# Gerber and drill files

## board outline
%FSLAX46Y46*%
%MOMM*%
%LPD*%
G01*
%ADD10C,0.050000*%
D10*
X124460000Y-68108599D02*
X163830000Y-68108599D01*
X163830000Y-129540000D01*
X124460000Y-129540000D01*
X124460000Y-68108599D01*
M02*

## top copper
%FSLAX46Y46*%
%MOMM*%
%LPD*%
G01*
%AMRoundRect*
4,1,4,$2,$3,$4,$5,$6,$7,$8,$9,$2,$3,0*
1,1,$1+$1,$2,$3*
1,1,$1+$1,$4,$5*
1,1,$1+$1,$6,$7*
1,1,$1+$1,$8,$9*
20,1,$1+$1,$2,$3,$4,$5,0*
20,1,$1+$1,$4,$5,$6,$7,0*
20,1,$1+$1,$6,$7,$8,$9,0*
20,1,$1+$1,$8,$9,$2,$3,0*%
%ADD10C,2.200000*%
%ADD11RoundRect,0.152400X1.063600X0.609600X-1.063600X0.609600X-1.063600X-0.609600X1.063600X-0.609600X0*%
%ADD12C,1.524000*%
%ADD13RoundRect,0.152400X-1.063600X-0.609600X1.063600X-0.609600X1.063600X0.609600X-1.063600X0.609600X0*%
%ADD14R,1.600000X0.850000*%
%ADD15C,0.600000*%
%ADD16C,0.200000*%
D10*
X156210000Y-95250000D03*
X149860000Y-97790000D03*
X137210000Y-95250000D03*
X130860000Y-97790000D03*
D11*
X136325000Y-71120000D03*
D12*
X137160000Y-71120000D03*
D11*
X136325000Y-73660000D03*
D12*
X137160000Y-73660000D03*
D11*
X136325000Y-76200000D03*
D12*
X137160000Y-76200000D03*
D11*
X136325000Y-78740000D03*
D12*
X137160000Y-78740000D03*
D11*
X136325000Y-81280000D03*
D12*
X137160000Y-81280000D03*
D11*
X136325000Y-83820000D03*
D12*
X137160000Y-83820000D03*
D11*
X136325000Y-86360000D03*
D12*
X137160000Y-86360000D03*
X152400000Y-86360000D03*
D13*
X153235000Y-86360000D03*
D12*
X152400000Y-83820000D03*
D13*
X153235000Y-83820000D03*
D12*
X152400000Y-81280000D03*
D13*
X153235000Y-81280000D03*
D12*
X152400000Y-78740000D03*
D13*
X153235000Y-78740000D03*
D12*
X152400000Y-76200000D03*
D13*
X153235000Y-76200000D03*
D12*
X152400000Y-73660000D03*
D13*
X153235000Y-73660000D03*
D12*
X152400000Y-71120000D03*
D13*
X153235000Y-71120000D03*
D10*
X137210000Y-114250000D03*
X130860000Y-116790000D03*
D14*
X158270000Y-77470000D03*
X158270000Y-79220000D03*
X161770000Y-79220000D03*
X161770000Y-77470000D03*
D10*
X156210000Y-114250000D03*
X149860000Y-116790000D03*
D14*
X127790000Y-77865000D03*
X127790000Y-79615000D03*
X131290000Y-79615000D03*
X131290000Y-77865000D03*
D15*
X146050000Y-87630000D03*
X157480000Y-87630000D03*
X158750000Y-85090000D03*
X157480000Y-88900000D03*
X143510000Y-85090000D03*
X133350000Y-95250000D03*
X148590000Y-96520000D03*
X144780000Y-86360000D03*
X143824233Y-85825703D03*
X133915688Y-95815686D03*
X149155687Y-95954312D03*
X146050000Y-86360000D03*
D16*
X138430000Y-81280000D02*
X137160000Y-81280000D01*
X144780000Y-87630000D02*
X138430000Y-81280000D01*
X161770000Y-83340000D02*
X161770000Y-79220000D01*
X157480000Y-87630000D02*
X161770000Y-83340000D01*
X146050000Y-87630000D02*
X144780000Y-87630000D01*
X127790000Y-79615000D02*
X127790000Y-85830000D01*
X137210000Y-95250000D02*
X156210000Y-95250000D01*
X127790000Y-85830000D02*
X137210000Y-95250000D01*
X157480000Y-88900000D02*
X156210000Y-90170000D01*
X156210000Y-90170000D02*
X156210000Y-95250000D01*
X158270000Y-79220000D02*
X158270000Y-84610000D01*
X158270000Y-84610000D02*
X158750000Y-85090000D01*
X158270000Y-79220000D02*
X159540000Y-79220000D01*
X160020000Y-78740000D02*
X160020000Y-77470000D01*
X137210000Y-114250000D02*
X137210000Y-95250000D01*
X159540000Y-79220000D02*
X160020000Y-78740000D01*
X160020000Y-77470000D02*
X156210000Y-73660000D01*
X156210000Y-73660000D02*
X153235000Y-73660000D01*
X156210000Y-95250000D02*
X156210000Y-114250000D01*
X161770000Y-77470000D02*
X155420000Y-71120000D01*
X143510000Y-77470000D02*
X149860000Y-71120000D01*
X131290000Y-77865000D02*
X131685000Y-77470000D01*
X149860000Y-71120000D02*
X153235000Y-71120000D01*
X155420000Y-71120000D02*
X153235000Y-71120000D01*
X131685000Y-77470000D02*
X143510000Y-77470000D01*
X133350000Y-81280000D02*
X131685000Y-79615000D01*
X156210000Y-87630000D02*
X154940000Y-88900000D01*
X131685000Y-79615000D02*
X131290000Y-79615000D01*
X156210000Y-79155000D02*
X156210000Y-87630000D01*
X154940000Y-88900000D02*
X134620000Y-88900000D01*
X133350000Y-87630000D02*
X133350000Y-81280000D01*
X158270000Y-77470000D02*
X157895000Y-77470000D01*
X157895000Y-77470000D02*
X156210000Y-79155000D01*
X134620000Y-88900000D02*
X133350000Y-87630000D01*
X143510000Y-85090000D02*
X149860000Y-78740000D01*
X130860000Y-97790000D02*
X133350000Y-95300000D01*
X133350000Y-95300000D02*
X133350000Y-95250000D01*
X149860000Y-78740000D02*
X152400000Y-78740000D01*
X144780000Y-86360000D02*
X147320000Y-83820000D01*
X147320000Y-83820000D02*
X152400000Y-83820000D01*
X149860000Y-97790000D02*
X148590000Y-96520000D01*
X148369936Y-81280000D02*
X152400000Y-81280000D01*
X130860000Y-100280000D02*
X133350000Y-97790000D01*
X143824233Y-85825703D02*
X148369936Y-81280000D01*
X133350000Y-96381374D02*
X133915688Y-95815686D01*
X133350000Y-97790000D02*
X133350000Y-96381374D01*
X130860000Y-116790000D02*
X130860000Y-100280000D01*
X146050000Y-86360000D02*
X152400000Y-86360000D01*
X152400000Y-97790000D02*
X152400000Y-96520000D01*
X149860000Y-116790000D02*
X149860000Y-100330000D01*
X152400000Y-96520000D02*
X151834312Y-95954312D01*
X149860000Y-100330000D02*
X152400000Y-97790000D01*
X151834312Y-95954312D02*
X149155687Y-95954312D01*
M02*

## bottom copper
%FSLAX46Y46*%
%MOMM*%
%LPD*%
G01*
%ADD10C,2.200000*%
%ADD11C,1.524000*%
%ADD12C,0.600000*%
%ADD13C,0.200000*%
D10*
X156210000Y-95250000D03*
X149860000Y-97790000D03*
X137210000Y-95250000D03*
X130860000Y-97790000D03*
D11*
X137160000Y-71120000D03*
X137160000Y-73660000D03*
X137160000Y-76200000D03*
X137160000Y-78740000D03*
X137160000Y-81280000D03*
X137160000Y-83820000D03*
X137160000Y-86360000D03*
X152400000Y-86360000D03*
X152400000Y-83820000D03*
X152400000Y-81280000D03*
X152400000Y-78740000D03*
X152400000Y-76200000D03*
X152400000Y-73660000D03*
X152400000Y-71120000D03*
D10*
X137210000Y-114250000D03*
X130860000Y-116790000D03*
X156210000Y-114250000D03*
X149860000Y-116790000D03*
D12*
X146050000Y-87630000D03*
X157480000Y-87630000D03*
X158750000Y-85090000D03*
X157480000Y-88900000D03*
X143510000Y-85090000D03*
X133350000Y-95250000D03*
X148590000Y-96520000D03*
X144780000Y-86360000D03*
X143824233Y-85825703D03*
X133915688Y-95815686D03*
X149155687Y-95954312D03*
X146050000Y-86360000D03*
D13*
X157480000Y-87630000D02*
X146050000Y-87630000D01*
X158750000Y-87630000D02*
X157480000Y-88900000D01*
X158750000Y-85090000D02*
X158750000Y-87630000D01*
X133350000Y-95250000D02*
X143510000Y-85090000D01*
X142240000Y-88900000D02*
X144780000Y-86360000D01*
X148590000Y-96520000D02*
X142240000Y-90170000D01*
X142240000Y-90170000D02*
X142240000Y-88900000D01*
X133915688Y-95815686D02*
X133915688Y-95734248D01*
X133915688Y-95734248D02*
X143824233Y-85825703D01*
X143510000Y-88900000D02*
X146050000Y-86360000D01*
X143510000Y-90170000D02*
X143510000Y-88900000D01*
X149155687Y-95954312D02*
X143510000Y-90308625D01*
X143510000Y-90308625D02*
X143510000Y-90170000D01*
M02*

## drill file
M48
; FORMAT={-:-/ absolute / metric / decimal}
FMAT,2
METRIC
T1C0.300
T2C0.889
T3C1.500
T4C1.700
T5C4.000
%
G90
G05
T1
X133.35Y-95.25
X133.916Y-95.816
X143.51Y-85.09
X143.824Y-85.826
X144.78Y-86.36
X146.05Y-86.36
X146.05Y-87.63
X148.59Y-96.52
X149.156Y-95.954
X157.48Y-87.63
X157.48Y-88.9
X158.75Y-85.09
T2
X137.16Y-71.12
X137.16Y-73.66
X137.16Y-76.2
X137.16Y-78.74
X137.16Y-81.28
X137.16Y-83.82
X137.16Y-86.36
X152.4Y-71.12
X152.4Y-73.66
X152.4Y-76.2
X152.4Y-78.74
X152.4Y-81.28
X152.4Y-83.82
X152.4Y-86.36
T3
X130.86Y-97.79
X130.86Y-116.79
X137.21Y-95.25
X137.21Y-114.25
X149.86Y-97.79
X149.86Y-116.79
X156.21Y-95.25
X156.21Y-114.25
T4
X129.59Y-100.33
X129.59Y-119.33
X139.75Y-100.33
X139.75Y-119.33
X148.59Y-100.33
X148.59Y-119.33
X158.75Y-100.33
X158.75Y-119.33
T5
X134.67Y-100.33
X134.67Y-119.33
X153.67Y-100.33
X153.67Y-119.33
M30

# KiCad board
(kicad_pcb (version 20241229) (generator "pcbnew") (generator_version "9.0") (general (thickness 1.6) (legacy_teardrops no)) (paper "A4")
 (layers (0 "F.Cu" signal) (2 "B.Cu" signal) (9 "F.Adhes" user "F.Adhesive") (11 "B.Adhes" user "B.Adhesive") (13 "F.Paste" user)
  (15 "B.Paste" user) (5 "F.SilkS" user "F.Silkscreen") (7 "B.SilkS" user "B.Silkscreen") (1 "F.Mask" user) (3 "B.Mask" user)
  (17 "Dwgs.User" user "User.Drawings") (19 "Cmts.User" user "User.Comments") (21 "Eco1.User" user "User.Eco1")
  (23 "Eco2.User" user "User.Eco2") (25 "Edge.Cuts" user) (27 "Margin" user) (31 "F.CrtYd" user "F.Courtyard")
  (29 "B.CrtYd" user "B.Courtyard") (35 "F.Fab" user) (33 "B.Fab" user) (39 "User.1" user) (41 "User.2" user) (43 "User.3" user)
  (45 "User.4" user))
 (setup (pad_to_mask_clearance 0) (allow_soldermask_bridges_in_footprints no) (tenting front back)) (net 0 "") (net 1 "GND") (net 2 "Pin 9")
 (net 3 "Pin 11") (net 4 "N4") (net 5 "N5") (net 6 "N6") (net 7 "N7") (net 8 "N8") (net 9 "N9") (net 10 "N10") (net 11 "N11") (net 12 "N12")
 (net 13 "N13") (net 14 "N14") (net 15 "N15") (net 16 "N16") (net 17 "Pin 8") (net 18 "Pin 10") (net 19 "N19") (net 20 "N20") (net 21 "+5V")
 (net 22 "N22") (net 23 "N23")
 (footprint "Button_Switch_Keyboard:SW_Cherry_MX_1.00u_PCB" (layer "F.Cu") (at 156.21 95.25)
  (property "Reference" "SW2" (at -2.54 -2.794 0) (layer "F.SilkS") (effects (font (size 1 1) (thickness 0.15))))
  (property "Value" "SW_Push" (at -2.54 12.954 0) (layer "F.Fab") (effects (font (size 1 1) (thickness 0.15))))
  (pad "" np_thru_hole circle (at -7.62 5.08) (size 1.7 1.7) (drill 1.7) (layers "*.Cu" "*.Mask"))
  (pad "" np_thru_hole circle (at -2.54 5.08) (size 4 4) (drill 4) (layers "*.Cu" "*.Mask"))
  (pad "" np_thru_hole circle (at 2.54 5.08) (size 1.7 1.7) (drill 1.7) (layers "*.Cu" "*.Mask"))
  (pad "1" thru_hole circle (at 0 0) (size 2.2 2.2) (drill 1.5) (layers "*.Cu" "*.Mask") (remove_unused_layers no) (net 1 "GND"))
  (pad "2" thru_hole circle (at -6.35 2.54) (size 2.2 2.2) (drill 1.5) (layers "*.Cu" "*.Mask") (remove_unused_layers no) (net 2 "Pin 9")))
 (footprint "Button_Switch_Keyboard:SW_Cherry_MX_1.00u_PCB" (layer "F.Cu") (at 137.21 95.25)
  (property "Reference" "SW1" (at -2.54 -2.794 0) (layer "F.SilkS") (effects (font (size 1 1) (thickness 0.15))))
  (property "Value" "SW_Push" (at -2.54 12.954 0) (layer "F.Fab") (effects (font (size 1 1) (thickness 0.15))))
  (pad "" np_thru_hole circle (at -7.62 5.08) (size 1.7 1.7) (drill 1.7) (layers "*.Cu" "*.Mask"))
  (pad "" np_thru_hole circle (at -2.54 5.08) (size 4 4) (drill 4) (layers "*.Cu" "*.Mask"))
  (pad "" np_thru_hole circle (at 2.54 5.08) (size 1.7 1.7) (drill 1.7) (layers "*.Cu" "*.Mask"))
  (pad "1" thru_hole circle (at 0 0) (size 2.2 2.2) (drill 1.5) (layers "*.Cu" "*.Mask") (remove_unused_layers no) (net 1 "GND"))
  (pad "2" thru_hole circle (at -6.35 2.54) (size 2.2 2.2) (drill 1.5) (layers "*.Cu" "*.Mask") (remove_unused_layers no) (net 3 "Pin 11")))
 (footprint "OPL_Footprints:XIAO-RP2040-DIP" (layer "F.Cu") (at 144.78 78.74)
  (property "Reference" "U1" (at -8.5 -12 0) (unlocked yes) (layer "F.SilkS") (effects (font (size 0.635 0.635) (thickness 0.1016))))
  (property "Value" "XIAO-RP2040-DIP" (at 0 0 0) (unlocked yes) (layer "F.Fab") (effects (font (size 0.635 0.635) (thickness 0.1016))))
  (pad "1" smd roundrect (at -8.455 -7.62 180) (size 2.432 1.524) (layers "F.Cu" "F.Mask") (roundrect_rratio 0.1) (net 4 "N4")
   (thermal_bridge_angle 45))
  (pad "1" thru_hole circle (at -7.62 -7.62 180) (size 1.524 1.524) (drill 0.889) (layers "*.Cu" "*.Mask") (remove_unused_layers no)
   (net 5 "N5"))
  (pad "2" smd roundrect (at -8.455 -5.08 180) (size 2.432 1.524) (layers "F.Cu" "F.Mask") (roundrect_rratio 0.1) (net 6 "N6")
   (thermal_bridge_angle 45))
  (pad "2" thru_hole circle (at -7.62 -5.08 180) (size 1.524 1.524) (drill 0.889) (layers "*.Cu" "*.Mask") (remove_unused_layers no)
   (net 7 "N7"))
  (pad "3" smd roundrect (at -8.455 -2.54 180) (size 2.432 1.524) (layers "F.Cu" "F.Mask") (roundrect_rratio 0.1) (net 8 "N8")
   (thermal_bridge_angle 45))
  (pad "3" thru_hole circle (at -7.62 -2.54 180) (size 1.524 1.524) (drill 0.889) (layers "*.Cu" "*.Mask") (remove_unused_layers no)
   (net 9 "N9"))
  (pad "4" smd roundrect (at -8.455 0 180) (size 2.432 1.524) (layers "F.Cu" "F.Mask") (roundrect_rratio 0.1) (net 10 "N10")
   (thermal_bridge_angle 45))
  (pad "4" thru_hole circle (at -7.62 0 180) (size 1.524 1.524) (drill 0.889) (layers "*.Cu" "*.Mask") (remove_unused_layers no)
   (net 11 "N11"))
  (pad "5" smd roundrect (at -8.455 2.54 180) (size 2.432 1.524) (layers "F.Cu" "F.Mask") (roundrect_rratio 0.1) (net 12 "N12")
   (thermal_bridge_angle 45))
  (pad "5" thru_hole circle (at -7.62 2.54 180) (size 1.524 1.524) (drill 0.889) (layers "*.Cu" "*.Mask") (remove_unused_layers no)
   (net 12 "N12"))
  (pad "6" smd roundrect (at -8.455 5.08 180) (size 2.432 1.524) (layers "F.Cu" "F.Mask") (roundrect_rratio 0.1) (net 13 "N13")
   (thermal_bridge_angle 45))
  (pad "6" thru_hole circle (at -7.62 5.08 180) (size 1.524 1.524) (drill 0.889) (layers "*.Cu" "*.Mask") (remove_unused_layers no)
   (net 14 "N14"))
  (pad "7" smd roundrect (at -8.455 7.62 180) (size 2.432 1.524) (layers "F.Cu" "F.Mask") (roundrect_rratio 0.1) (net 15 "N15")
   (thermal_bridge_angle 45))
  (pad "7" thru_hole circle (at -7.62 7.62 180) (size 1.524 1.524) (drill 0.889) (layers "*.Cu" "*.Mask") (remove_unused_layers no)
   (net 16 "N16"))
  (pad "8" thru_hole circle (at 7.62 7.62) (size 1.524 1.524) (drill 0.889) (layers "*.Cu" "*.Mask") (remove_unused_layers no)
   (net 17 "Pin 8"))
  (pad "8" smd roundrect (at 8.455 7.62) (size 2.432 1.524) (layers "F.Cu" "F.Mask") (roundrect_rratio 0.1) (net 17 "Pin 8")
   (thermal_bridge_angle 45))
  (pad "9" thru_hole circle (at 7.62 5.08) (size 1.524 1.524) (drill 0.889) (layers "*.Cu" "*.Mask") (remove_unused_layers no)
   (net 2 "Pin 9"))
  (pad "9" smd roundrect (at 8.455 5.08) (size 2.432 1.524) (layers "F.Cu" "F.Mask") (roundrect_rratio 0.1) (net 2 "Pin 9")
   (thermal_bridge_angle 45))
  (pad "10" thru_hole circle (at 7.62 2.54) (size 1.524 1.524) (drill 0.889) (layers "*.Cu" "*.Mask") (remove_unused_layers no)
   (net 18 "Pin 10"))
  (pad "10" smd roundrect (at 8.455 2.54) (size 2.432 1.524) (layers "F.Cu" "F.Mask") (roundrect_rratio 0.1) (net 18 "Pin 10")
   (thermal_bridge_angle 45))
  (pad "11" thru_hole circle (at 7.62 0) (size 1.524 1.524) (drill 0.889) (layers "*.Cu" "*.Mask") (remove_unused_layers no)
   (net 3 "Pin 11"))
  (pad "11" smd roundrect (at 8.455 0) (size 2.432 1.524) (layers "F.Cu" "F.Mask") (roundrect_rratio 0.1) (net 3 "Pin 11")
   (thermal_bridge_angle 45))
  (pad "12" thru_hole circle (at 7.62 -2.54) (size 1.524 1.524) (drill 0.889) (layers "*.Cu" "*.Mask") (remove_unused_layers no)
   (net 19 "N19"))
  (pad "12" smd roundrect (at 8.455 -2.54) (size 2.432 1.524) (layers "F.Cu" "F.Mask") (roundrect_rratio 0.1) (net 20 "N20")
   (thermal_bridge_angle 45))
  (pad "13" thru_hole circle (at 7.62 -5.08) (size 1.524 1.524) (drill 0.889) (layers "*.Cu" "*.Mask") (remove_unused_layers no)
   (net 1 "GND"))
  (pad "13" smd roundrect (at 8.455 -5.08) (size 2.432 1.524) (layers "F.Cu" "F.Mask") (roundrect_rratio 0.1) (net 1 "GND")
   (thermal_bridge_angle 45))
  (pad "14" thru_hole circle (at 7.62 -7.62) (size 1.524 1.524) (drill 0.889) (layers "*.Cu" "*.Mask") (remove_unused_layers no)
   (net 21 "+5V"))
  (pad "14" smd roundrect (at 8.455 -7.62) (size 2.432 1.524) (layers "F.Cu" "F.Mask") (roundrect_rratio 0.1) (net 21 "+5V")
   (thermal_bridge_angle 45)))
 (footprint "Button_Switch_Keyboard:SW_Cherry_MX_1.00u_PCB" (layer "F.Cu") (at 137.21 114.25)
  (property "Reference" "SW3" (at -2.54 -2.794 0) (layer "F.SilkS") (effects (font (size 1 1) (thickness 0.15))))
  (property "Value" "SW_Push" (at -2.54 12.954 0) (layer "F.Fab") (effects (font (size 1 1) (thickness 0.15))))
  (pad "" np_thru_hole circle (at -7.62 5.08) (size 1.7 1.7) (drill 1.7) (layers "*.Cu" "*.Mask"))
  (pad "" np_thru_hole circle (at -2.54 5.08) (size 4 4) (drill 4) (layers "*.Cu" "*.Mask"))
  (pad "" np_thru_hole circle (at 2.54 5.08) (size 1.7 1.7) (drill 1.7) (layers "*.Cu" "*.Mask"))
  (pad "1" thru_hole circle (at 0 0) (size 2.2 2.2) (drill 1.5) (layers "*.Cu" "*.Mask") (remove_unused_layers no) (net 1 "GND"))
  (pad "2" thru_hole circle (at -6.35 2.54) (size 2.2 2.2) (drill 1.5) (layers "*.Cu" "*.Mask") (remove_unused_layers no) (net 18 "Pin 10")))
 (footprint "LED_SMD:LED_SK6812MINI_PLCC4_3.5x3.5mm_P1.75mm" (layer "F.Cu") (at 160.02 78.345)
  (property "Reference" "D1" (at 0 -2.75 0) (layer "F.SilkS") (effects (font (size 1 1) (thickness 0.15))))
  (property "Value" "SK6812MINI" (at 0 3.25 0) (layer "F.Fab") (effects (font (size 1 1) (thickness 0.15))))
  (pad "1" smd rect (at -1.75 -0.875) (size 1.6 0.85) (layers "F.Cu" "F.Mask" "F.Paste") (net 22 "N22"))
  (pad "2" smd rect (at -1.75 0.875) (size 1.6 0.85) (layers "F.Cu" "F.Mask" "F.Paste") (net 1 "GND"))
  (pad "3" smd rect (at 1.75 0.875) (size 1.6 0.85) (layers "F.Cu" "F.Mask" "F.Paste") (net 12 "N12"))
  (pad "4" smd rect (at 1.75 -0.875) (size 1.6 0.85) (layers "F.Cu" "F.Mask" "F.Paste") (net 21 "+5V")))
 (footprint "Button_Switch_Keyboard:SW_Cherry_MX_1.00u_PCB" (layer "F.Cu") (at 156.21 114.25)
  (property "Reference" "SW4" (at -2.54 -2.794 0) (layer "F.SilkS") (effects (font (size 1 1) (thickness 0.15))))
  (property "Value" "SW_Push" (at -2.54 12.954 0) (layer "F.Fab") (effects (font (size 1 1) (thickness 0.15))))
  (pad "" np_thru_hole circle (at -7.62 5.08) (size 1.7 1.7) (drill 1.7) (layers "*.Cu" "*.Mask"))
  (pad "" np_thru_hole circle (at -2.54 5.08) (size 4 4) (drill 4) (layers "*.Cu" "*.Mask"))
  (pad "" np_thru_hole circle (at 2.54 5.08) (size 1.7 1.7) (drill 1.7) (layers "*.Cu" "*.Mask"))
  (pad "1" thru_hole circle (at 0 0) (size 2.2 2.2) (drill 1.5) (layers "*.Cu" "*.Mask") (remove_unused_layers no) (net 1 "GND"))
  (pad "2" thru_hole circle (at -6.35 2.54) (size 2.2 2.2) (drill 1.5) (layers "*.Cu" "*.Mask") (remove_unused_layers no) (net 17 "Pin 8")))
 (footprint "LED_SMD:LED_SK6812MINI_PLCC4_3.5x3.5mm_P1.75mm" (layer "F.Cu") (at 129.54 78.74)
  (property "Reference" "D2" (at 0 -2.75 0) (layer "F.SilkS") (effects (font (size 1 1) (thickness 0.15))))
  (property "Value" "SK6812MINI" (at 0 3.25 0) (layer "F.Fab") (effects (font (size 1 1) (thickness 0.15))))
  (pad "1" smd rect (at -1.75 -0.875) (size 1.6 0.85) (layers "F.Cu" "F.Mask" "F.Paste") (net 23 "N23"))
  (pad "2" smd rect (at -1.75 0.875) (size 1.6 0.85) (layers "F.Cu" "F.Mask" "F.Paste") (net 1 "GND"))
  (pad "3" smd rect (at 1.75 0.875) (size 1.6 0.85) (layers "F.Cu" "F.Mask" "F.Paste") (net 22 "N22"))
  (pad "4" smd rect (at 1.75 -0.875) (size 1.6 0.85) (layers "F.Cu" "F.Mask" "F.Paste") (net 21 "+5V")))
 (gr_rect (start 124.46 68.108599) (end 163.83 129.54) (stroke (width 0.05) (type default)) (fill no) (layer "Edge.Cuts"))
 (segment (start 138.43 81.28) (end 137.16 81.28) (width 0.2) (layer "F.Cu") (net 12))
 (segment (start 144.78 87.63) (end 138.43 81.28) (width 0.2) (layer "F.Cu") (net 12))
 (segment (start 161.77 83.34) (end 161.77 79.22) (width 0.2) (layer "F.Cu") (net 12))
 (segment (start 157.48 87.63) (end 161.77 83.34) (width 0.2) (layer "F.Cu") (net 12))
 (segment (start 146.05 87.63) (end 144.78 87.63) (width 0.2) (layer "F.Cu") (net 12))
 (via (at 146.05 87.63) (size 0.6) (drill 0.3) (layers "F.Cu" "B.Cu") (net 12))
 (via (at 157.48 87.63) (size 0.6) (drill 0.3) (layers "F.Cu" "B.Cu") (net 12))
 (segment (start 157.48 87.63) (end 146.05 87.63) (width 0.2) (layer "B.Cu") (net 12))
 (segment (start 127.79 79.615) (end 127.79 85.83) (width 0.2) (layer "F.Cu") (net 1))
 (segment (start 137.21 95.25) (end 156.21 95.25) (width 0.2) (layer "F.Cu") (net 1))
 (segment (start 127.79 85.83) (end 137.21 95.25) (width 0.2) (layer "F.Cu") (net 1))
 (segment (start 157.48 88.9) (end 156.21 90.17) (width 0.2) (layer "F.Cu") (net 1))
 (segment (start 156.21 90.17) (end 156.21 95.25) (width 0.2) (layer "F.Cu") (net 1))
 (segment (start 158.27 79.22) (end 158.27 84.61) (width 0.2) (layer "F.Cu") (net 1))
 (segment (start 158.27 84.61) (end 158.75 85.09) (width 0.2) (layer "F.Cu") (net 1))
 (segment (start 158.27 79.22) (end 159.54 79.22) (width 0.2) (layer "F.Cu") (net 1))
 (segment (start 160.02 78.74) (end 160.02 77.47) (width 0.2) (layer "F.Cu") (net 1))
 (segment (start 137.21 114.25) (end 137.21 95.25) (width 0.2) (layer "F.Cu") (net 1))
 (segment (start 159.54 79.22) (end 160.02 78.74) (width 0.2) (layer "F.Cu") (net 1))
 (segment (start 160.02 77.47) (end 156.21 73.66) (width 0.2) (layer "F.Cu") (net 1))
 (segment (start 156.21 73.66) (end 153.235 73.66) (width 0.2) (layer "F.Cu") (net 1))
 (segment (start 156.21 95.25) (end 156.21 114.25) (width 0.2) (layer "F.Cu") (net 1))
 (via (at 158.75 85.09) (size 0.6) (drill 0.3) (layers "F.Cu" "B.Cu") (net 1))
 (via (at 157.48 88.9) (size 0.6) (drill 0.3) (layers "F.Cu" "B.Cu") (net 1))
 (segment (start 158.75 87.63) (end 157.48 88.9) (width 0.2) (layer "B.Cu") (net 1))
 (segment (start 158.75 85.09) (end 158.75 87.63) (width 0.2) (layer "B.Cu") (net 1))
 (segment (start 161.77 77.47) (end 155.42 71.12) (width 0.2) (layer "F.Cu") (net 21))
 (segment (start 143.51 77.47) (end 149.86 71.12) (width 0.2) (layer "F.Cu") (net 21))
 (segment (start 131.29 77.865) (end 131.685 77.47) (width 0.2) (layer "F.Cu") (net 21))
 (segment (start 149.86 71.12) (end 153.235 71.12) (width 0.2) (layer "F.Cu") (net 21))
 (segment (start 155.42 71.12) (end 153.235 71.12) (width 0.2) (layer "F.Cu") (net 21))
 (segment (start 131.685 77.47) (end 143.51 77.47) (width 0.2) (layer "F.Cu") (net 21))
 (segment (start 133.35 81.28) (end 131.685 79.615) (width 0.2) (layer "F.Cu") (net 22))
 (segment (start 156.21 87.63) (end 154.94 88.9) (width 0.2) (layer "F.Cu") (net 22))
 (segment (start 131.685 79.615) (end 131.29 79.615) (width 0.2) (layer "F.Cu") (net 22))
 (segment (start 156.21 79.155) (end 156.21 87.63) (width 0.2) (layer "F.Cu") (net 22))
 (segment (start 154.94 88.9) (end 134.62 88.9) (width 0.2) (layer "F.Cu") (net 22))
 (segment (start 133.35 87.63) (end 133.35 81.28) (width 0.2) (layer "F.Cu") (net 22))
 (segment (start 158.27 77.47) (end 157.895 77.47) (width 0.2) (layer "F.Cu") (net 22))
 (segment (start 157.895 77.47) (end 156.21 79.155) (width 0.2) (layer "F.Cu") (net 22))
 (segment (start 134.62 88.9) (end 133.35 87.63) (width 0.2) (layer "F.Cu") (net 22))
 (segment (start 143.51 85.09) (end 149.86 78.74) (width 0.2) (layer "F.Cu") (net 3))
 (segment (start 130.86 97.79) (end 133.35 95.3) (width 0.2) (layer "F.Cu") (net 3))
 (segment (start 133.35 95.3) (end 133.35 95.25) (width 0.2) (layer "F.Cu") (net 3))
 (segment (start 149.86 78.74) (end 152.4 78.74) (width 0.2) (layer "F.Cu") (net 3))
 (via (at 143.51 85.09) (size 0.6) (drill 0.3) (layers "F.Cu" "B.Cu") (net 3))
 (via (at 133.35 95.25) (size 0.6) (drill 0.3) (layers "F.Cu" "B.Cu") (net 3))
 (segment (start 133.35 95.25) (end 143.51 85.09) (width 0.2) (layer "B.Cu") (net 3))
 (segment (start 144.78 86.36) (end 147.32 83.82) (width 0.2) (layer "F.Cu") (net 2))
 (segment (start 147.32 83.82) (end 152.4 83.82) (width 0.2) (layer "F.Cu") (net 2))
 (segment (start 149.86 97.79) (end 148.59 96.52) (width 0.2) (layer "F.Cu") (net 2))
 (via (at 148.59 96.52) (size 0.6) (drill 0.3) (layers "F.Cu" "B.Cu") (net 2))
 (via (at 144.78 86.36) (size 0.6) (drill 0.3) (layers "F.Cu" "B.Cu") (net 2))
 (segment (start 142.24 88.9) (end 144.78 86.36) (width 0.2) (layer "B.Cu") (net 2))
 (segment (start 148.59 96.52) (end 142.24 90.17) (width 0.2) (layer "B.Cu") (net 2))
 (segment (start 142.24 90.17) (end 142.24 88.9) (width 0.2) (layer "B.Cu") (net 2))
 (segment (start 148.369936 81.28) (end 152.4 81.28) (width 0.2) (layer "F.Cu") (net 18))
 (segment (start 130.86 100.28) (end 133.35 97.79) (width 0.2) (layer "F.Cu") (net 18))
 (segment (start 143.824233 85.825703) (end 148.369936 81.28) (width 0.2) (layer "F.Cu") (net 18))
 (segment (start 133.35 96.381374) (end 133.915688 95.815686) (width 0.2) (layer "F.Cu") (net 18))
 (segment (start 133.35 97.79) (end 133.35 96.381374) (width 0.2) (layer "F.Cu") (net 18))
 (segment (start 130.86 116.79) (end 130.86 100.28) (width 0.2) (layer "F.Cu") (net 18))
 (via (at 143.824233 85.825703) (size 0.6) (drill 0.3) (layers "F.Cu" "B.Cu") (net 18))
 (via (at 133.915688 95.815686) (size 0.6) (drill 0.3) (layers "F.Cu" "B.Cu") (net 18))
 (segment (start 133.915688 95.815686) (end 133.915688 95.734248) (width 0.2) (layer "B.Cu") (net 18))
 (segment (start 133.915688 95.734248) (end 143.824233 85.825703) (width 0.2) (layer "B.Cu") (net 18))
 (segment (start 146.05 86.36) (end 152.4 86.36) (width 0.2) (layer "F.Cu") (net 17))
 (segment (start 152.4 97.79) (end 152.4 96.52) (width 0.2) (layer "F.Cu") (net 17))
 (segment (start 149.86 116.79) (end 149.86 100.33) (width 0.2) (layer "F.Cu") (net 17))
 (segment (start 152.4 96.52) (end 151.834312 95.954312) (width 0.2) (layer "F.Cu") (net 17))
 (segment (start 149.86 100.33) (end 152.4 97.79) (width 0.2) (layer "F.Cu") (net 17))
 (segment (start 151.834312 95.954312) (end 149.155687 95.954312) (width 0.2) (layer "F.Cu") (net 17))
 (via (at 149.155687 95.954312) (size 0.6) (drill 0.3) (layers "F.Cu" "B.Cu") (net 17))
 (via (at 146.05 86.36) (size 0.6) (drill 0.3) (layers "F.Cu" "B.Cu") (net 17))
 (segment (start 143.51 88.9) (end 146.05 86.36) (width 0.2) (layer "B.Cu") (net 17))
 (segment (start 143.51 90.17) (end 143.51 88.9) (width 0.2) (layer "B.Cu") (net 17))
 (segment (start 149.155687 95.954312) (end 143.51 90.308625) (width 0.2) (layer "B.Cu") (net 17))
 (segment (start 143.51 90.308625) (end 143.51 90.17) (width 0.2) (layer "B.Cu") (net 17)))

